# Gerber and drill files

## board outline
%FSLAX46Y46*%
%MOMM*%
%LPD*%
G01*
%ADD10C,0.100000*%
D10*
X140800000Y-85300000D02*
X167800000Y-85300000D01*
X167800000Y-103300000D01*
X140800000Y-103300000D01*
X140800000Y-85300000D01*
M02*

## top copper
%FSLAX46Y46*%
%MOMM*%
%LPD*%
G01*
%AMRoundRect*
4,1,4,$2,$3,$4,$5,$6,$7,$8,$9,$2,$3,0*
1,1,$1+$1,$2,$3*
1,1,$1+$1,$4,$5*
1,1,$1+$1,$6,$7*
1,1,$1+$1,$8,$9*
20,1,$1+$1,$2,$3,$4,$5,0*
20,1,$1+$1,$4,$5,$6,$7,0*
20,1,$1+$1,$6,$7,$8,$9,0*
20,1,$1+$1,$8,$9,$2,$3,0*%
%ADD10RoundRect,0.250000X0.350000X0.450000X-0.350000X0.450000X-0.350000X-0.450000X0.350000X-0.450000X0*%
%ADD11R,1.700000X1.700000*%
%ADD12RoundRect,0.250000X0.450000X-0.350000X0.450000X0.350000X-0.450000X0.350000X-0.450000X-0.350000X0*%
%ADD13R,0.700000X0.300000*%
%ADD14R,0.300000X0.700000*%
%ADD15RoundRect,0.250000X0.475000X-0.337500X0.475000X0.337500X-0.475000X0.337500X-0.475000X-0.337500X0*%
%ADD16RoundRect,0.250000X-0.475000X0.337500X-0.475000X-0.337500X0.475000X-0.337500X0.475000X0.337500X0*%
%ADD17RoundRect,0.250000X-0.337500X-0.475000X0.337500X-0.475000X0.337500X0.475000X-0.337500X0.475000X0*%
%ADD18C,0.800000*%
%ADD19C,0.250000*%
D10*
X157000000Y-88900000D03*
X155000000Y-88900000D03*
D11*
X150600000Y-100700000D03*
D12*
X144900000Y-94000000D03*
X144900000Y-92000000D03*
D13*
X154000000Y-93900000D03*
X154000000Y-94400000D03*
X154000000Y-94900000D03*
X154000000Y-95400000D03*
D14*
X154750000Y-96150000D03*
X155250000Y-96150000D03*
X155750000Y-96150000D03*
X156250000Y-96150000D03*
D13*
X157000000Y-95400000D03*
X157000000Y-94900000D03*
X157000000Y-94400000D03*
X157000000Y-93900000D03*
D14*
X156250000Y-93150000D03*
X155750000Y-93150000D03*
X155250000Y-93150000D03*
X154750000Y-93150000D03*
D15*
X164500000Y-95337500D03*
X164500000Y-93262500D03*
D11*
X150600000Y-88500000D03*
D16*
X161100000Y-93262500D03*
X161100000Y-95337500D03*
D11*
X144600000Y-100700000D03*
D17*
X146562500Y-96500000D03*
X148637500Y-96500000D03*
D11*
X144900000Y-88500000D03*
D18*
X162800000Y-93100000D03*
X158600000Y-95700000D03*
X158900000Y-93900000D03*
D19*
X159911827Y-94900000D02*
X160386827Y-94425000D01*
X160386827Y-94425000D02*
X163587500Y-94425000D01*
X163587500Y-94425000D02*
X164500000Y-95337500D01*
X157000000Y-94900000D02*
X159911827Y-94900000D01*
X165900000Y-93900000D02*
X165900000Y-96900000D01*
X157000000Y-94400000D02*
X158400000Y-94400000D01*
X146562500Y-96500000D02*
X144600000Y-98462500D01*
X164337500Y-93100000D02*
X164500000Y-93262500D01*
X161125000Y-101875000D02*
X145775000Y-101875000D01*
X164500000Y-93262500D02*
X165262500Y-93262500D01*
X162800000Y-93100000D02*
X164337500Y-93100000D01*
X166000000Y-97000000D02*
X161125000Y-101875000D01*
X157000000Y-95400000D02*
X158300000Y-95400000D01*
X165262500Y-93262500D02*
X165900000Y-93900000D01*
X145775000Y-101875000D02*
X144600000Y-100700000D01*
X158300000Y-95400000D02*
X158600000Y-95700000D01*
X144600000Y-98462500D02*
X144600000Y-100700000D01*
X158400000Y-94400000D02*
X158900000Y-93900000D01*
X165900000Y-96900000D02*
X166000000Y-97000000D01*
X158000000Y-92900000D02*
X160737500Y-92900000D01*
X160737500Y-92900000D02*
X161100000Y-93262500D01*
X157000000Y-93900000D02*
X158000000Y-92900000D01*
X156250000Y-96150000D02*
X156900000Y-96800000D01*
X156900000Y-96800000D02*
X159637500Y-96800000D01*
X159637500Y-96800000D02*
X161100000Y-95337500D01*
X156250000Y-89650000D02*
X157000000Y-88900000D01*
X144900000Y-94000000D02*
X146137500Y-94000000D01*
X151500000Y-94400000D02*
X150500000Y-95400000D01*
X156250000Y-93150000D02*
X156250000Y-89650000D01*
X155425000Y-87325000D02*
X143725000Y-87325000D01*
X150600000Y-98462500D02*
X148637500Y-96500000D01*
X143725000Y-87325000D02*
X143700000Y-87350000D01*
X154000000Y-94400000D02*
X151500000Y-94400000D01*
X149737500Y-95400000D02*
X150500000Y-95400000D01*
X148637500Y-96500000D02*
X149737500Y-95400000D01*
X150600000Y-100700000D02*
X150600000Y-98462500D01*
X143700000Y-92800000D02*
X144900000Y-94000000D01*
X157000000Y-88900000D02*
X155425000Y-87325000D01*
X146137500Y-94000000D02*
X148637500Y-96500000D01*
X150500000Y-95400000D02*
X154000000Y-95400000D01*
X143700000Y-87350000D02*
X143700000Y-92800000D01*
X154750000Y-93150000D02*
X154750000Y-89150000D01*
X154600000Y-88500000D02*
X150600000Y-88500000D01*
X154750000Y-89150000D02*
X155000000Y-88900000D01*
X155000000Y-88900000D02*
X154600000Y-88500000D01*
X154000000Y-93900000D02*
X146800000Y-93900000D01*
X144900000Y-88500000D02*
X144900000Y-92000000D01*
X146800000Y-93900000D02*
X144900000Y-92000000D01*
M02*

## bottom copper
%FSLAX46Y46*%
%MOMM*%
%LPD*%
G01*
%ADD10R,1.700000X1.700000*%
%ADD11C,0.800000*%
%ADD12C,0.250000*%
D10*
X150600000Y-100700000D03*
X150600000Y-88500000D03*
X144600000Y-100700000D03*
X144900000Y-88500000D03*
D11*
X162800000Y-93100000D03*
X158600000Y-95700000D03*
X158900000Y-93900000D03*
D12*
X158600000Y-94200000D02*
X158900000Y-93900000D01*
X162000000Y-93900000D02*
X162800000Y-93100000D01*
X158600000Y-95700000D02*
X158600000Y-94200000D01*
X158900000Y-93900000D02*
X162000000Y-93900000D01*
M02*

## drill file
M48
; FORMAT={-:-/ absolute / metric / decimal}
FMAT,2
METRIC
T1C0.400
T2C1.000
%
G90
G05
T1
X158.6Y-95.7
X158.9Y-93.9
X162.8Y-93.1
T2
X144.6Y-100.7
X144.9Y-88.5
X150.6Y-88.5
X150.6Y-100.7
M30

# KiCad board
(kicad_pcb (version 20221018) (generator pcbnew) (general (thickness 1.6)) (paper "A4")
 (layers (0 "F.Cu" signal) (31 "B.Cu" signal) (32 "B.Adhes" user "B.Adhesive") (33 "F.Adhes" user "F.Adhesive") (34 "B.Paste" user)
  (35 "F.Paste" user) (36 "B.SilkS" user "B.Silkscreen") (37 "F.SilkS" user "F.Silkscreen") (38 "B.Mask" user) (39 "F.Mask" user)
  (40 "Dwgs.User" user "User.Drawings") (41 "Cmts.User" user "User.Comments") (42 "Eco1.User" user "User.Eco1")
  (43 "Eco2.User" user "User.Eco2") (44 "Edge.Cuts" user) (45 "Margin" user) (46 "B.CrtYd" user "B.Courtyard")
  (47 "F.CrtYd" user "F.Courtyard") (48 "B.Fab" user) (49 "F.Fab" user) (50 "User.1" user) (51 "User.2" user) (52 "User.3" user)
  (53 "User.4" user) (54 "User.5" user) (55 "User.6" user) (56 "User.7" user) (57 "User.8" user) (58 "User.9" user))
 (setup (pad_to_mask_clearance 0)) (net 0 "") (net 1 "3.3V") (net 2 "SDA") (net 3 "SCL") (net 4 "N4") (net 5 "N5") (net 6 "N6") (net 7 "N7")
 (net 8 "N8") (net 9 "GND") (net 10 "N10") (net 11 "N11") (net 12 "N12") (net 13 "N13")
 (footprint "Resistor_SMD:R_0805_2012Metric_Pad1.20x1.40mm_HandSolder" (layer "F.Cu") (at 156 88.9 180)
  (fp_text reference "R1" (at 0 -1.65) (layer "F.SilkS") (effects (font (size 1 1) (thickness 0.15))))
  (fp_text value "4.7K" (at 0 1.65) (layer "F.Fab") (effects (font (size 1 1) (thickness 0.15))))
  (pad "1" smd roundrect (at -1 0 180) (size 1.2 1.4) (layers "F.Cu" "F.Paste" "F.Mask") (roundrect_rratio 0.208333) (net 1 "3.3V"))
  (pad "2" smd roundrect (at 1 0 180) (size 1.2 1.4) (layers "F.Cu" "F.Paste" "F.Mask") (roundrect_rratio 0.208333) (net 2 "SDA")))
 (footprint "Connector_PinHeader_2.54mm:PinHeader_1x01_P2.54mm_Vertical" (layer "F.Cu") (at 150.6 100.7)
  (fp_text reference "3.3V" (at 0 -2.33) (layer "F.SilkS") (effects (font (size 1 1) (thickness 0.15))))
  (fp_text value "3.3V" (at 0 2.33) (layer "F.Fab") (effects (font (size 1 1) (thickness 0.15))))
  (pad "1" thru_hole rect (at 0 0) (size 1.7 1.7) (drill 1) (layers "*.Cu" "*.Mask") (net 1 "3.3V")))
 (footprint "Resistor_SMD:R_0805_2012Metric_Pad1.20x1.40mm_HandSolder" (layer "F.Cu") (at 144.9 93 90)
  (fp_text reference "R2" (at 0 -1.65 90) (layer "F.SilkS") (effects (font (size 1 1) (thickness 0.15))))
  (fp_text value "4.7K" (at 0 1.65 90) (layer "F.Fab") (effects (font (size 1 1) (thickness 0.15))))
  (pad "1" smd roundrect (at -1 0 90) (size 1.2 1.4) (layers "F.Cu" "F.Paste" "F.Mask") (roundrect_rratio 0.208333) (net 1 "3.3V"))
  (pad "2" smd roundrect (at 1 0 90) (size 1.2 1.4) (layers "F.Cu" "F.Paste" "F.Mask") (roundrect_rratio 0.208333) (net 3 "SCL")))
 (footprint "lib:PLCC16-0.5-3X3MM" (layer "F.Cu") (at 154 96.15)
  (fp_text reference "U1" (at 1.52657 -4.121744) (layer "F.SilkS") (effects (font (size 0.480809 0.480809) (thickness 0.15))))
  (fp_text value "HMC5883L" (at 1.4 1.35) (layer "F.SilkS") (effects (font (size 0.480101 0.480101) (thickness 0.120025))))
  (pad "1" smd rect (at 0 -2.25) (size 0.7 0.3) (layers "F.Cu" "F.Paste" "F.Mask") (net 3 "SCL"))
  (pad "2" smd rect (at 0 -1.75) (size 0.7 0.3) (layers "F.Cu" "F.Paste" "F.Mask") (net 1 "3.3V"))
  (pad "3" smd rect (at 0 -1.25) (size 0.7 0.3) (layers "F.Cu" "F.Paste" "F.Mask") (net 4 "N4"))
  (pad "4" smd rect (at 0 -0.75) (size 0.7 0.3) (layers "F.Cu" "F.Paste" "F.Mask") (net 1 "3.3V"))
  (pad "5" smd rect (at 0.75 0 90) (size 0.7 0.3) (layers "F.Cu" "F.Paste" "F.Mask") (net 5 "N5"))
  (pad "6" smd rect (at 1.25 0 90) (size 0.7 0.3) (layers "F.Cu" "F.Paste" "F.Mask") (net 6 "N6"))
  (pad "7" smd rect (at 1.75 0 90) (size 0.7 0.3) (layers "F.Cu" "F.Paste" "F.Mask") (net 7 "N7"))
  (pad "8" smd rect (at 2.25 0 90) (size 0.7 0.3) (layers "F.Cu" "F.Paste" "F.Mask") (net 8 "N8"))
  (pad "9" smd rect (at 3 -0.75) (size 0.7 0.3) (layers "F.Cu" "F.Paste" "F.Mask") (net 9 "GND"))
  (pad "10" smd rect (at 3 -1.25) (size 0.7 0.3) (layers "F.Cu" "F.Paste" "F.Mask") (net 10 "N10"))
  (pad "11" smd rect (at 3 -1.75) (size 0.7 0.3) (layers "F.Cu" "F.Paste" "F.Mask") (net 9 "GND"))
  (pad "12" smd rect (at 3 -2.25) (size 0.7 0.3) (layers "F.Cu" "F.Paste" "F.Mask") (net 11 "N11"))
  (pad "13" smd rect (at 2.25 -3 90) (size 0.7 0.3) (layers "F.Cu" "F.Paste" "F.Mask") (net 1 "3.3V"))
  (pad "14" smd rect (at 1.75 -3 90) (size 0.7 0.3) (layers "F.Cu" "F.Paste" "F.Mask") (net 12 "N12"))
  (pad "15" smd rect (at 1.25 -3 90) (size 0.7 0.3) (layers "F.Cu" "F.Paste" "F.Mask") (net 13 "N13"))
  (pad "16" smd rect (at 0.75 -3 90) (size 0.7 0.3) (layers "F.Cu" "F.Paste" "F.Mask") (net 2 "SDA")))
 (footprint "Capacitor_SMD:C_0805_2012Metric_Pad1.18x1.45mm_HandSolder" (layer "F.Cu") (at 164.5 94.3 90)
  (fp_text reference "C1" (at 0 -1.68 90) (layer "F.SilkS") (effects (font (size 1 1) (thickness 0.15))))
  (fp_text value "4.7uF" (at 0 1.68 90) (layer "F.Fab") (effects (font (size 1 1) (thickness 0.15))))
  (pad "1" smd roundrect (at -1.0375 0 90) (size 1.175 1.45) (layers "F.Cu" "F.Paste" "F.Mask") (roundrect_rratio 0.212766) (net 10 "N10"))
  (pad "2" smd roundrect (at 1.0375 0 90) (size 1.175 1.45) (layers "F.Cu" "F.Paste" "F.Mask") (roundrect_rratio 0.212766) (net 9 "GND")))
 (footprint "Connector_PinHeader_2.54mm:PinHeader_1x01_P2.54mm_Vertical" (layer "F.Cu") (at 150.6 88.5)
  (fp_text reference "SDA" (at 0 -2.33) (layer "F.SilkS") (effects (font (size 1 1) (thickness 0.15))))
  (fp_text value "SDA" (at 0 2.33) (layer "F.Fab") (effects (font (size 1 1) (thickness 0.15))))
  (pad "1" thru_hole rect (at 0 0) (size 1.7 1.7) (drill 1) (layers "*.Cu" "*.Mask") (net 2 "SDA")))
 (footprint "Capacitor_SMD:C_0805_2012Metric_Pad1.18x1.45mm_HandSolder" (layer "F.Cu") (at 161.1 94.3 -90)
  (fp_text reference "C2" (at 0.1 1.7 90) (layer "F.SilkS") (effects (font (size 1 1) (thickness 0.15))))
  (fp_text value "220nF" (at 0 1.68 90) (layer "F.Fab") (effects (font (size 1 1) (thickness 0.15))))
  (pad "1" smd roundrect (at -1.0375 0 270) (size 1.175 1.45) (layers "F.Cu" "F.Paste" "F.Mask") (roundrect_rratio 0.212766) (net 11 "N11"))
  (pad "2" smd roundrect (at 1.0375 0 270) (size 1.175 1.45) (layers "F.Cu" "F.Paste" "F.Mask") (roundrect_rratio 0.212766) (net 8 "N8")))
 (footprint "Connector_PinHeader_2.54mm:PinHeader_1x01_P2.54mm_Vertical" (layer "F.Cu") (at 144.6 100.7)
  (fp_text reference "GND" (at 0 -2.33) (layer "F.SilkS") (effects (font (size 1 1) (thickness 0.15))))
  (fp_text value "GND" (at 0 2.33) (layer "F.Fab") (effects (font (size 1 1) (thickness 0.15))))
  (pad "1" thru_hole rect (at 0 0) (size 1.7 1.7) (drill 1) (layers "*.Cu" "*.Mask") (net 9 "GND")))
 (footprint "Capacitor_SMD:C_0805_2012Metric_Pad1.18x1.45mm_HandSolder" (layer "F.Cu") (at 147.6 96.5)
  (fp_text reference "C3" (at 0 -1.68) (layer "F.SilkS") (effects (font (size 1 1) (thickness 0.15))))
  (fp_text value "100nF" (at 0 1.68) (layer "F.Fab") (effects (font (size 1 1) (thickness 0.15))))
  (pad "1" smd roundrect (at -1.0375 0) (size 1.175 1.45) (layers "F.Cu" "F.Paste" "F.Mask") (roundrect_rratio 0.212766) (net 9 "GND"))
  (pad "2" smd roundrect (at 1.0375 0) (size 1.175 1.45) (layers "F.Cu" "F.Paste" "F.Mask") (roundrect_rratio 0.212766) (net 1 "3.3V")))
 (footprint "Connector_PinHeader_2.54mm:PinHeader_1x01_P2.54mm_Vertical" (layer "F.Cu") (at 144.9 88.5)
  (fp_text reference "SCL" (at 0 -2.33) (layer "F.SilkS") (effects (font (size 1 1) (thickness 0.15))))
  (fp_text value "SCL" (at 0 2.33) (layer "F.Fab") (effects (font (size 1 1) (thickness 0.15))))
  (pad "1" thru_hole rect (at 0 0) (size 1.7 1.7) (drill 1) (layers "*.Cu" "*.Mask") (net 3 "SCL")))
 (gr_rect (start 140.8 85.3) (end 167.8 103.3) (stroke (width 0.1) (type default)) (fill none) (layer "Edge.Cuts"))
 (segment (start 159.911827 94.9) (end 160.386827 94.425) (width 0.25) (layer "F.Cu") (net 10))
 (segment (start 160.386827 94.425) (end 163.5875 94.425) (width 0.25) (layer "F.Cu") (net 10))
 (segment (start 163.5875 94.425) (end 164.5 95.3375) (width 0.25) (layer "F.Cu") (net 10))
 (segment (start 157 94.9) (end 159.911827 94.9) (width 0.25) (layer "F.Cu") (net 10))
 (segment (start 165.9 93.9) (end 165.9 96.9) (width 0.25) (layer "F.Cu") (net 9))
 (segment (start 157 94.4) (end 158.4 94.4) (width 0.25) (layer "F.Cu") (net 9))
 (segment (start 146.5625 96.5) (end 144.6 98.4625) (width 0.25) (layer "F.Cu") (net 9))
 (segment (start 164.3375 93.1) (end 164.5 93.2625) (width 0.25) (layer "F.Cu") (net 9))
 (segment (start 161.125 101.875) (end 145.775 101.875) (width 0.25) (layer "F.Cu") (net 9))
 (segment (start 164.5 93.2625) (end 165.2625 93.2625) (width 0.25) (layer "F.Cu") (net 9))
 (segment (start 162.8 93.1) (end 164.3375 93.1) (width 0.25) (layer "F.Cu") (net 9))
 (segment (start 166 97) (end 161.125 101.875) (width 0.25) (layer "F.Cu") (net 9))
 (segment (start 157 95.4) (end 158.3 95.4) (width 0.25) (layer "F.Cu") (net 9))
 (segment (start 165.2625 93.2625) (end 165.9 93.9) (width 0.25) (layer "F.Cu") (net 9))
 (segment (start 145.775 101.875) (end 144.6 100.7) (width 0.25) (layer "F.Cu") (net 9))
 (segment (start 158.3 95.4) (end 158.6 95.7) (width 0.25) (layer "F.Cu") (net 9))
 (segment (start 144.6 98.4625) (end 144.6 100.7) (width 0.25) (layer "F.Cu") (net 9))
 (segment (start 158.4 94.4) (end 158.9 93.9) (width 0.25) (layer "F.Cu") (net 9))
 (segment (start 165.9 96.9) (end 166 97) (width 0.25) (layer "F.Cu") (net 9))
 (via (at 162.8 93.1) (size 0.8) (drill 0.4) (layers "F.Cu" "B.Cu") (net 9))
 (via (at 158.6 95.7) (size 0.8) (drill 0.4) (layers "F.Cu" "B.Cu") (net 9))
 (via (at 158.9 93.9) (size 0.8) (drill 0.4) (layers "F.Cu" "B.Cu") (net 9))
 (segment (start 158.6 94.2) (end 158.9 93.9) (width 0.25) (layer "B.Cu") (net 9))
 (segment (start 162 93.9) (end 162.8 93.1) (width 0.25) (layer "B.Cu") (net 9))
 (segment (start 158.6 95.7) (end 158.6 94.2) (width 0.25) (layer "B.Cu") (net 9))
 (segment (start 158.9 93.9) (end 162 93.9) (width 0.25) (layer "B.Cu") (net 9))
 (segment (start 158 92.9) (end 160.7375 92.9) (width 0.25) (layer "F.Cu") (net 11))
 (segment (start 160.7375 92.9) (end 161.1 93.2625) (width 0.25) (layer "F.Cu") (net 11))
 (segment (start 157 93.9) (end 158 92.9) (width 0.25) (layer "F.Cu") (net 11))
 (segment (start 156.25 96.15) (end 156.9 96.8) (width 0.25) (layer "F.Cu") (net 8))
 (segment (start 156.9 96.8) (end 159.6375 96.8) (width 0.25) (layer "F.Cu") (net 8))
 (segment (start 159.6375 96.8) (end 161.1 95.3375) (width 0.25) (layer "F.Cu") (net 8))
 (segment (start 156.25 89.65) (end 157 88.9) (width 0.25) (layer "F.Cu") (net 1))
 (segment (start 144.9 94) (end 146.1375 94) (width 0.25) (layer "F.Cu") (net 1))
 (segment (start 151.5 94.4) (end 150.5 95.4) (width 0.25) (layer "F.Cu") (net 1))
 (segment (start 156.25 93.15) (end 156.25 89.65) (width 0.25) (layer "F.Cu") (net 1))
 (segment (start 155.425 87.325) (end 143.725 87.325) (width 0.25) (layer "F.Cu") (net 1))
 (segment (start 150.6 98.4625) (end 148.6375 96.5) (width 0.25) (layer "F.Cu") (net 1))
 (segment (start 143.725 87.325) (end 143.7 87.35) (width 0.25) (layer "F.Cu") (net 1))
 (segment (start 154 94.4) (end 151.5 94.4) (width 0.25) (layer "F.Cu") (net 1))
 (segment (start 149.7375 95.4) (end 150.5 95.4) (width 0.25) (layer "F.Cu") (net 1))
 (segment (start 148.6375 96.5) (end 149.7375 95.4) (width 0.25) (layer "F.Cu") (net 1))
 (segment (start 150.6 100.7) (end 150.6 98.4625) (width 0.25) (layer "F.Cu") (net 1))
 (segment (start 143.7 92.8) (end 144.9 94) (width 0.25) (layer "F.Cu") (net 1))
 (segment (start 157 88.9) (end 155.425 87.325) (width 0.25) (layer "F.Cu") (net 1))
 (segment (start 146.1375 94) (end 148.6375 96.5) (width 0.25) (layer "F.Cu") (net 1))
 (segment (start 150.5 95.4) (end 154 95.4) (width 0.25) (layer "F.Cu") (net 1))
 (segment (start 143.7 87.35) (end 143.7 92.8) (width 0.25) (layer "F.Cu") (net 1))
 (segment (start 154.75 93.15) (end 154.75 89.15) (width 0.25) (layer "F.Cu") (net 2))
 (segment (start 154.6 88.5) (end 150.6 88.5) (width 0.25) (layer "F.Cu") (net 2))
 (segment (start 154.75 89.15) (end 155 88.9) (width 0.25) (layer "F.Cu") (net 2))
 (segment (start 155 88.9) (end 154.6 88.5) (width 0.25) (layer "F.Cu") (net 2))
 (segment (start 154 93.9) (end 146.8 93.9) (width 0.25) (layer "F.Cu") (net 3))
 (segment (start 144.9 88.5) (end 144.9 92) (width 0.25) (layer "F.Cu") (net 3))
 (segment (start 146.8 93.9) (end 144.9 92) (width 0.25) (layer "F.Cu") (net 3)))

